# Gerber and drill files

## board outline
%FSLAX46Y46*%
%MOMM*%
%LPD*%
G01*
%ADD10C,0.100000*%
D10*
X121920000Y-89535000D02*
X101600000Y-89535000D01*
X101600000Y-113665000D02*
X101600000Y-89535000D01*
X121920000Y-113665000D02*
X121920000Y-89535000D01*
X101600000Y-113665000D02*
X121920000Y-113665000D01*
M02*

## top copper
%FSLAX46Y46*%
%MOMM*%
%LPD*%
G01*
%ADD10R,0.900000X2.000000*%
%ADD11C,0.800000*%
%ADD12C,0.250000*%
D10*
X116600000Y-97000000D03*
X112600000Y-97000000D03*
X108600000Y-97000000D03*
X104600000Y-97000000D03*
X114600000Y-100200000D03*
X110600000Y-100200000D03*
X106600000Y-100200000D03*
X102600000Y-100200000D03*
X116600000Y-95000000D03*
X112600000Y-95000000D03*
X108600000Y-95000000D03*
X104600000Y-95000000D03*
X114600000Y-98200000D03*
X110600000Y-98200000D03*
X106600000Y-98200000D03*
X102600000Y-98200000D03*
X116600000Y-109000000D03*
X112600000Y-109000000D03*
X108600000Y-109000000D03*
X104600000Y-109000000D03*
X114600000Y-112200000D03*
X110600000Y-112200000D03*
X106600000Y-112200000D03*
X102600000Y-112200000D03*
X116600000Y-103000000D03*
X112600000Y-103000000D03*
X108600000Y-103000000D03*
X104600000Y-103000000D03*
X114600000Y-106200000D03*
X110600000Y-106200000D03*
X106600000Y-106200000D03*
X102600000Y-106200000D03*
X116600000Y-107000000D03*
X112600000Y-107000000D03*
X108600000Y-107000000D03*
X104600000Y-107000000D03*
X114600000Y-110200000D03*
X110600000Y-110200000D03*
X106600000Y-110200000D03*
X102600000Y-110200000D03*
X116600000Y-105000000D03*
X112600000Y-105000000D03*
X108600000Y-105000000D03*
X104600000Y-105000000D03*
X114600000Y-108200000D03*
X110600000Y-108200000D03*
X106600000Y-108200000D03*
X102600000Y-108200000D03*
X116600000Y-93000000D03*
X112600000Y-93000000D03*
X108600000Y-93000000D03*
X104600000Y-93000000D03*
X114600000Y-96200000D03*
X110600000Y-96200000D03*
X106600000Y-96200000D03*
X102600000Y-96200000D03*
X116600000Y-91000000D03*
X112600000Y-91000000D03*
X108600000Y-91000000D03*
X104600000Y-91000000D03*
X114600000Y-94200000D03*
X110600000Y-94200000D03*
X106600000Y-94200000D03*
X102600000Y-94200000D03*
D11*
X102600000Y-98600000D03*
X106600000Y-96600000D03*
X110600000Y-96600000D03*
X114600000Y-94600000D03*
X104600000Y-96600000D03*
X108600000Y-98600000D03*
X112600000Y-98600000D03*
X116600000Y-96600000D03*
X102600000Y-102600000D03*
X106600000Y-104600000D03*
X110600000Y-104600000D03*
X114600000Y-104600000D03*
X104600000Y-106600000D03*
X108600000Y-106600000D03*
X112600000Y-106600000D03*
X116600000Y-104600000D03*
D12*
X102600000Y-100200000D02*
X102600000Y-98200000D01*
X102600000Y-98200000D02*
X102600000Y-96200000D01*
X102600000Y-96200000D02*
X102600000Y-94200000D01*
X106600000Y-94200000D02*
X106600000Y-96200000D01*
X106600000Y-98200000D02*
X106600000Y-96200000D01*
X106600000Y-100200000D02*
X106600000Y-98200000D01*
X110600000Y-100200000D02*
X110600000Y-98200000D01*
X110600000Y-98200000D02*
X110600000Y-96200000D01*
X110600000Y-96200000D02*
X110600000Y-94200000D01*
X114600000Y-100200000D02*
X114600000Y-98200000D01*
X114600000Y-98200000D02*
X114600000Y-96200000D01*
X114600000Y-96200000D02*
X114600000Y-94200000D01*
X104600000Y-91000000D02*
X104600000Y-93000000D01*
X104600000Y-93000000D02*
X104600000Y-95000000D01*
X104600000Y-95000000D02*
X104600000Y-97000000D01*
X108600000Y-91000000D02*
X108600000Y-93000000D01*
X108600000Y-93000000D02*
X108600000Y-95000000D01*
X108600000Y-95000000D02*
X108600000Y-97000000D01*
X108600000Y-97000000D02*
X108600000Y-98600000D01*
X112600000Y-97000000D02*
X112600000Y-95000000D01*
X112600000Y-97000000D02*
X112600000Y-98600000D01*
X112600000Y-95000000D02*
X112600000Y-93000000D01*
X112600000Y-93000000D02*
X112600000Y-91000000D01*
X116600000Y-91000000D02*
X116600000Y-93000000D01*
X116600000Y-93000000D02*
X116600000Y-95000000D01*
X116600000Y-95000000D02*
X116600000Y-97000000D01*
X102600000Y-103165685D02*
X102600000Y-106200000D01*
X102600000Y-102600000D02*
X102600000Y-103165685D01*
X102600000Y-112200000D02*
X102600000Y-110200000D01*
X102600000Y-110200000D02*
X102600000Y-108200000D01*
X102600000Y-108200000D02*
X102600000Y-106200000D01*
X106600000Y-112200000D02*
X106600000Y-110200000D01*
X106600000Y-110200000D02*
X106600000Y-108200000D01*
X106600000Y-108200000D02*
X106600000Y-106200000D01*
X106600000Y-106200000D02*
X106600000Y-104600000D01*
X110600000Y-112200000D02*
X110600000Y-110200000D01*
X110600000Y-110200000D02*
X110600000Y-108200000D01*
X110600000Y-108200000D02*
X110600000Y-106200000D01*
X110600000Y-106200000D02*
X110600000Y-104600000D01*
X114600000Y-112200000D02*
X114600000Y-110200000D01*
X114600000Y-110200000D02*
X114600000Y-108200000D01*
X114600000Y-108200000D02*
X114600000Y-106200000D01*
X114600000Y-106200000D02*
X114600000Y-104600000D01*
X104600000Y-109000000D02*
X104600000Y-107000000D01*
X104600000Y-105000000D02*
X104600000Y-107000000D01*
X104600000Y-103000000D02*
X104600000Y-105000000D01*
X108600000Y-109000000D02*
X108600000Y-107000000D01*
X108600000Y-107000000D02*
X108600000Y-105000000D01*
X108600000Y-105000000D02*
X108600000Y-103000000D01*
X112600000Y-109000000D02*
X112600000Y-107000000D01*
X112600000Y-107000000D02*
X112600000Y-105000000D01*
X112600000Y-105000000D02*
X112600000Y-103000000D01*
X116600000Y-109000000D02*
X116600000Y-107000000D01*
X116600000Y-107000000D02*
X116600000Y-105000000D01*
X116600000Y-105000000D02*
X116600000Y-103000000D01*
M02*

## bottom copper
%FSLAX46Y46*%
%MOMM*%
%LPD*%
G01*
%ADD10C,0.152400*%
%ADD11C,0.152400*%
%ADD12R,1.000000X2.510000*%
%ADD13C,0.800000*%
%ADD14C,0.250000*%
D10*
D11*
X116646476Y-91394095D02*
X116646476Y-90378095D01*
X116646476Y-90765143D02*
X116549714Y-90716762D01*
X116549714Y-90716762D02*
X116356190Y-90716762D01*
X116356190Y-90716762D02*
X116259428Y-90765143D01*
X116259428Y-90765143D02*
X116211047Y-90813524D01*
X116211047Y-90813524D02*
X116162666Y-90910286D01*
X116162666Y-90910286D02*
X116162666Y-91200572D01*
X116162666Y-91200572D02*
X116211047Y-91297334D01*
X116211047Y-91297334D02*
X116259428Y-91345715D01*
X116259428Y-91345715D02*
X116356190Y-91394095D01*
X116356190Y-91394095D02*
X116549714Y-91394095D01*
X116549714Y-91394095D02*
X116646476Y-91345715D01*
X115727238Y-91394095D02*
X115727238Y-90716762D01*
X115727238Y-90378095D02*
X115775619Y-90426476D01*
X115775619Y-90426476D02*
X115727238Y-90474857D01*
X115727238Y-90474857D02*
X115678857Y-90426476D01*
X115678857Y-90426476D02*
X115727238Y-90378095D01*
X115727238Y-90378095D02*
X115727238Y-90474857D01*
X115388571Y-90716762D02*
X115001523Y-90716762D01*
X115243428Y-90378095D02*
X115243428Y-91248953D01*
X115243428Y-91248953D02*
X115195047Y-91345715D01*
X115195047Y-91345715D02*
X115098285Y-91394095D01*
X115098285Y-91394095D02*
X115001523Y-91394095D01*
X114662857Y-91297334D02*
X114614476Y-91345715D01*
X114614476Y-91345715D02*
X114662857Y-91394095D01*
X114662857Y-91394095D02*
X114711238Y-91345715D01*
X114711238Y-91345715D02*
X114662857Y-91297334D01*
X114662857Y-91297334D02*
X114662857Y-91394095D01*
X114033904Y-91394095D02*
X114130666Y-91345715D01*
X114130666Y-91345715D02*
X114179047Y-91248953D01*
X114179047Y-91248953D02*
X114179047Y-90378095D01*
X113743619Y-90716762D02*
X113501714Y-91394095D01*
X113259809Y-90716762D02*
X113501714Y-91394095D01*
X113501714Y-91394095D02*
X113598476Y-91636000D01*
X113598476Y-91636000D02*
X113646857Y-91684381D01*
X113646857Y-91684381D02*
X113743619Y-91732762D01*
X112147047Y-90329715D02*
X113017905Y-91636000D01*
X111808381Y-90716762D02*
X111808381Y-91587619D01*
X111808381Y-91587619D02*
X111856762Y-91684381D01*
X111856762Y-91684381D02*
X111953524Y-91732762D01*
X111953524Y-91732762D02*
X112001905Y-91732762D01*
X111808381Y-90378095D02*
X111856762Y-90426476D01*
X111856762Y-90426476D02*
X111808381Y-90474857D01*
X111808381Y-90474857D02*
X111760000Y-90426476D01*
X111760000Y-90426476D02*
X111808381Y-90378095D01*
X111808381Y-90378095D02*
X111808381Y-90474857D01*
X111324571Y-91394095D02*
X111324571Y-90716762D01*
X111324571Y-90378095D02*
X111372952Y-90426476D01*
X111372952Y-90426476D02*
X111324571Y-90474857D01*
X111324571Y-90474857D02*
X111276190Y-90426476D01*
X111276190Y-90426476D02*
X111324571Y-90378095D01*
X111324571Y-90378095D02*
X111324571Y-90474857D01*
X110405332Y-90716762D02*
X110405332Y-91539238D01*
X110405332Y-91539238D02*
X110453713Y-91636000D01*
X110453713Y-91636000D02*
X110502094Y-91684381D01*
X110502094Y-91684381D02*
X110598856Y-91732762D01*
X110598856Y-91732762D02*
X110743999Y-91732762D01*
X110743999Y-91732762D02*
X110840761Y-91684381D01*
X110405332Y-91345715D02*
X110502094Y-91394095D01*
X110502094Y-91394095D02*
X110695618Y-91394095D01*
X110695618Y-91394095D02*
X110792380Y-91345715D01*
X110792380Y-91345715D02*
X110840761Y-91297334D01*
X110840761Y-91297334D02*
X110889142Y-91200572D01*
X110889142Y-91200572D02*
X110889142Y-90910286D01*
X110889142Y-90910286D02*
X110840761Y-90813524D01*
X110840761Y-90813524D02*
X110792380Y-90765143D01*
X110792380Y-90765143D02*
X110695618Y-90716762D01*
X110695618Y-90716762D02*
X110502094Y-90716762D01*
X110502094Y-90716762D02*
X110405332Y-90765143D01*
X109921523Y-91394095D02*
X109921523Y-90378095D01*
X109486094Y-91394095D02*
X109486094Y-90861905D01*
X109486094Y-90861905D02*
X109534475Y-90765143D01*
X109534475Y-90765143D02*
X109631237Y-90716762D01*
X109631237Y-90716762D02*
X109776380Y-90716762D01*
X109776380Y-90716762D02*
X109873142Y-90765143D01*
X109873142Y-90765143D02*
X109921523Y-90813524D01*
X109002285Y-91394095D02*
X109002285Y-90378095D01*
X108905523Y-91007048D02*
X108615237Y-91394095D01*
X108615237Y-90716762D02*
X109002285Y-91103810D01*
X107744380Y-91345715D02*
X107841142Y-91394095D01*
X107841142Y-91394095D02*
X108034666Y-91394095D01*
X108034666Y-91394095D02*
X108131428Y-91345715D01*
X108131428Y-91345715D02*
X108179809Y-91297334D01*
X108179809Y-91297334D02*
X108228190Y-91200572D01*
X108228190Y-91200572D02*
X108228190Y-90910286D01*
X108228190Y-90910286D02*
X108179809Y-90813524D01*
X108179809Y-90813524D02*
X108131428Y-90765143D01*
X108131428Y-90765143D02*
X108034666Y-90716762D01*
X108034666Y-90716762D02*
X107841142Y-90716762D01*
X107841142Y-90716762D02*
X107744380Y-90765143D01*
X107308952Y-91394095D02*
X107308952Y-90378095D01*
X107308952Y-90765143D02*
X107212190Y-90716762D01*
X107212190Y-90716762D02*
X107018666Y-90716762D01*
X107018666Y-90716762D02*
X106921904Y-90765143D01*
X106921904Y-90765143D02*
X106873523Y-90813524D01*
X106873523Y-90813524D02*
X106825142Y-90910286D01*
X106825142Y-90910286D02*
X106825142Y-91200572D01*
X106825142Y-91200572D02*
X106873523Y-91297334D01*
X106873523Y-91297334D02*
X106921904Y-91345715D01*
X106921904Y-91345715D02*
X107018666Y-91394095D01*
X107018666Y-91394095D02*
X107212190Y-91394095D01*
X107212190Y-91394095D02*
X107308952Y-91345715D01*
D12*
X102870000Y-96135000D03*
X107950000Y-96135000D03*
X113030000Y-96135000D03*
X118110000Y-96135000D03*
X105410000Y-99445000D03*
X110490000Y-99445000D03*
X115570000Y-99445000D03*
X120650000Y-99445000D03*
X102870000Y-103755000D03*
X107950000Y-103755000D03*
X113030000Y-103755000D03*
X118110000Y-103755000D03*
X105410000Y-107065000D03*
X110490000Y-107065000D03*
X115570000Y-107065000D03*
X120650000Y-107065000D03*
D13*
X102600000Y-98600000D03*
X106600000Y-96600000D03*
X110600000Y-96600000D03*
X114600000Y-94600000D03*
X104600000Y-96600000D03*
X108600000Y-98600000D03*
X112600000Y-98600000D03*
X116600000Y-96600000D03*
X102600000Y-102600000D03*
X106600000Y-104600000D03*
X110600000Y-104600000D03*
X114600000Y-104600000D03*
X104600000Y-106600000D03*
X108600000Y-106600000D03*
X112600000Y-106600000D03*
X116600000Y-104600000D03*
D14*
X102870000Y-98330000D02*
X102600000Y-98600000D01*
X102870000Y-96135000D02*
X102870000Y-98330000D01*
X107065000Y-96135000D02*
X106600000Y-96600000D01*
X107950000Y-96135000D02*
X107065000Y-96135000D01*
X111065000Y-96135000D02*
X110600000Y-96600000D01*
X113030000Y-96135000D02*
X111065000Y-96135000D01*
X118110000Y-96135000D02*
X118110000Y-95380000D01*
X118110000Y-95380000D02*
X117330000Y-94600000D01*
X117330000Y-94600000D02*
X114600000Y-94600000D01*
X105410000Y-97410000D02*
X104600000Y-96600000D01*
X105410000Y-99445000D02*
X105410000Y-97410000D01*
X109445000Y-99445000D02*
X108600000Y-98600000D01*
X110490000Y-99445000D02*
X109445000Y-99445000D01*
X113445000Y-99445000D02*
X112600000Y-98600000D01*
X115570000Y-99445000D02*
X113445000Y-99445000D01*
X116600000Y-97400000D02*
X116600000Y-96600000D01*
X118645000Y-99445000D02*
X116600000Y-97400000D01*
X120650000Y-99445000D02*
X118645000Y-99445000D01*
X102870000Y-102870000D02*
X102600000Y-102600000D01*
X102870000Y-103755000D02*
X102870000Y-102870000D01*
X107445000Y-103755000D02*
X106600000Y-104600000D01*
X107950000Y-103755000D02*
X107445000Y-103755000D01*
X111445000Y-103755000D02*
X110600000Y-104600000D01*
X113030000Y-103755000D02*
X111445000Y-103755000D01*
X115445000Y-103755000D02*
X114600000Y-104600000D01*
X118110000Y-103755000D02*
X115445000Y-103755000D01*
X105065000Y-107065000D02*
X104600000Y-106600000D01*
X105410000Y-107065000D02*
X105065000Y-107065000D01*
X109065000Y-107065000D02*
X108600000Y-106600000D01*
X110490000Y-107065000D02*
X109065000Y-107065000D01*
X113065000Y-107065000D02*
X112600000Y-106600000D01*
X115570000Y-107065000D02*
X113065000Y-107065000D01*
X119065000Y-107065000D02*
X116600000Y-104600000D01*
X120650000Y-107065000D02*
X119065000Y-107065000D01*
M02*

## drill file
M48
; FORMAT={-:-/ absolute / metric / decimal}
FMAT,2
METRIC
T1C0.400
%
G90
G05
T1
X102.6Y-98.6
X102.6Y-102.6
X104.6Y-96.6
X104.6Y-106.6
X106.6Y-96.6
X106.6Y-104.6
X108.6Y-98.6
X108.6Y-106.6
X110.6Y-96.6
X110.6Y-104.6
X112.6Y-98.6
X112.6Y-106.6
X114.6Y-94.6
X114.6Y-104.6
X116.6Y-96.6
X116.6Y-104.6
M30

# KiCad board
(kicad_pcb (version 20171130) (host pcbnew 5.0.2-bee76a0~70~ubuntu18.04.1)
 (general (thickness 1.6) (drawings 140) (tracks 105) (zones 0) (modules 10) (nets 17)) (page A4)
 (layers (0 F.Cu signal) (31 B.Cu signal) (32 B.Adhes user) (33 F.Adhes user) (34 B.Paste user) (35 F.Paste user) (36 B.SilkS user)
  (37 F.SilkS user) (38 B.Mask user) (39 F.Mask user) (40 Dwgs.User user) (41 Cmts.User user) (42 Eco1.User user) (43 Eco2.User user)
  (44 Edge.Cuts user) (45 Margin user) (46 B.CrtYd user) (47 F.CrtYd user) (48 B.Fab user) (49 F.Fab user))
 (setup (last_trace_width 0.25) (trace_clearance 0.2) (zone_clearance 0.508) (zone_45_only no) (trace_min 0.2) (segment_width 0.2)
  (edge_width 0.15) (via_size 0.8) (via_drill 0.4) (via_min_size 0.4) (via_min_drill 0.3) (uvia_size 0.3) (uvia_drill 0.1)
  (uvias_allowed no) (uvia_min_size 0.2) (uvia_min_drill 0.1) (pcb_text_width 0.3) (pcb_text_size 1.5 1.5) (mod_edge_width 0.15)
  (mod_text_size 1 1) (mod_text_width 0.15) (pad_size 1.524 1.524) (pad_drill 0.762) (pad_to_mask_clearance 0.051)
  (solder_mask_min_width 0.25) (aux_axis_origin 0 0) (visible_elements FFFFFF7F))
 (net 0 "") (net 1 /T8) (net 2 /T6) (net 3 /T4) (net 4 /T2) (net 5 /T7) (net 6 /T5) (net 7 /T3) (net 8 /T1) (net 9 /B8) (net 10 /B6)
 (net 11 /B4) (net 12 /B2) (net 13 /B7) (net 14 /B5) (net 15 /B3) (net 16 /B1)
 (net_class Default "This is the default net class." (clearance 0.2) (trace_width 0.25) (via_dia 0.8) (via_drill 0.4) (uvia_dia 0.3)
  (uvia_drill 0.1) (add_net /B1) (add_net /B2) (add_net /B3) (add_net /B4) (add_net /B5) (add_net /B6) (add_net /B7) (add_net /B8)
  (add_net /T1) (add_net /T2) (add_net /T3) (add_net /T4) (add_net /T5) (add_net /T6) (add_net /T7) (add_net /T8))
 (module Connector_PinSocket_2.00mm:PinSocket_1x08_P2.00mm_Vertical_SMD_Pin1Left (layer F.Cu) (at 109.6 98.6 90)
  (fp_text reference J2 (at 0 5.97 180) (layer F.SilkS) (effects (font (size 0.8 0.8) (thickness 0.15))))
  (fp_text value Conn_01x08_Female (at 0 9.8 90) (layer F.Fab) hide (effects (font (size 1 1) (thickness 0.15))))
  (pad 8 smd rect (at 1.6 7 90) (size 2 0.9) (layers F.Cu F.Paste F.Mask) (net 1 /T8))
  (pad 6 smd rect (at 1.6 3 90) (size 2 0.9) (layers F.Cu F.Paste F.Mask) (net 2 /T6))
  (pad 4 smd rect (at 1.6 -1 90) (size 2 0.9) (layers F.Cu F.Paste F.Mask) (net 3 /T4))
  (pad 2 smd rect (at 1.6 -5 90) (size 2 0.9) (layers F.Cu F.Paste F.Mask) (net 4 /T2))
  (pad 7 smd rect (at -1.6 5 90) (size 2 0.9) (layers F.Cu F.Paste F.Mask) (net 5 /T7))
  (pad 5 smd rect (at -1.6 1 90) (size 2 0.9) (layers F.Cu F.Paste F.Mask) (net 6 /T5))
  (pad 3 smd rect (at -1.6 -3 90) (size 2 0.9) (layers F.Cu F.Paste F.Mask) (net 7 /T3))
  (pad 1 smd rect (at -1.6 -7 90) (size 2 0.9) (layers F.Cu F.Paste F.Mask) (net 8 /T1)))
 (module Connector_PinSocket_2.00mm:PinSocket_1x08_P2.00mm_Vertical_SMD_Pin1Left (layer F.Cu) (at 109.6 96.6 90)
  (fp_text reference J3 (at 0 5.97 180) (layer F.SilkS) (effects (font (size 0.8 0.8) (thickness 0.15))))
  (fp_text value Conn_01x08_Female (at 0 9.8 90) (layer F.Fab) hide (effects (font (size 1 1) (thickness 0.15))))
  (pad 8 smd rect (at 1.6 7 90) (size 2 0.9) (layers F.Cu F.Paste F.Mask) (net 1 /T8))
  (pad 6 smd rect (at 1.6 3 90) (size 2 0.9) (layers F.Cu F.Paste F.Mask) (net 2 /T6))
  (pad 4 smd rect (at 1.6 -1 90) (size 2 0.9) (layers F.Cu F.Paste F.Mask) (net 3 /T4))
  (pad 2 smd rect (at 1.6 -5 90) (size 2 0.9) (layers F.Cu F.Paste F.Mask) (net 4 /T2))
  (pad 7 smd rect (at -1.6 5 90) (size 2 0.9) (layers F.Cu F.Paste F.Mask) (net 5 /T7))
  (pad 5 smd rect (at -1.6 1 90) (size 2 0.9) (layers F.Cu F.Paste F.Mask) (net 6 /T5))
  (pad 3 smd rect (at -1.6 -3 90) (size 2 0.9) (layers F.Cu F.Paste F.Mask) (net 7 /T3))
  (pad 1 smd rect (at -1.6 -7 90) (size 2 0.9) (layers F.Cu F.Paste F.Mask) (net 8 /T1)))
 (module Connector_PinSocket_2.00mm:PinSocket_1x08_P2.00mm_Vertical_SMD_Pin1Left (layer F.Cu) (at 109.6 110.6 90)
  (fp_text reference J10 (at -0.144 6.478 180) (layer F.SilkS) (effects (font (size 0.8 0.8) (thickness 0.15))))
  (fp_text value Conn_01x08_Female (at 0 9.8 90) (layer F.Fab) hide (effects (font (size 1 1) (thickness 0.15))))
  (pad 8 smd rect (at 1.6 7 90) (size 2 0.9) (layers F.Cu F.Paste F.Mask) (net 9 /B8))
  (pad 6 smd rect (at 1.6 3 90) (size 2 0.9) (layers F.Cu F.Paste F.Mask) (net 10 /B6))
  (pad 4 smd rect (at 1.6 -1 90) (size 2 0.9) (layers F.Cu F.Paste F.Mask) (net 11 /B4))
  (pad 2 smd rect (at 1.6 -5 90) (size 2 0.9) (layers F.Cu F.Paste F.Mask) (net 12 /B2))
  (pad 7 smd rect (at -1.6 5 90) (size 2 0.9) (layers F.Cu F.Paste F.Mask) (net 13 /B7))
  (pad 5 smd rect (at -1.6 1 90) (size 2 0.9) (layers F.Cu F.Paste F.Mask) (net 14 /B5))
  (pad 3 smd rect (at -1.6 -3 90) (size 2 0.9) (layers F.Cu F.Paste F.Mask) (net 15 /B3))
  (pad 1 smd rect (at -1.6 -7 90) (size 2 0.9) (layers F.Cu F.Paste F.Mask) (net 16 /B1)))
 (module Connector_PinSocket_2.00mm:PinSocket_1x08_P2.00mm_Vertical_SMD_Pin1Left (layer F.Cu) (at 109.6 104.6 90)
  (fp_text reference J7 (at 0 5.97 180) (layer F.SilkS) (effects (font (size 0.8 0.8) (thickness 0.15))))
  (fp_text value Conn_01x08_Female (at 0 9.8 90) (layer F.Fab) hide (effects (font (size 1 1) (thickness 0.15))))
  (pad 8 smd rect (at 1.6 7 90) (size 2 0.9) (layers F.Cu F.Paste F.Mask) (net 9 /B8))
  (pad 6 smd rect (at 1.6 3 90) (size 2 0.9) (layers F.Cu F.Paste F.Mask) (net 10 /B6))
  (pad 4 smd rect (at 1.6 -1 90) (size 2 0.9) (layers F.Cu F.Paste F.Mask) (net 11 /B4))
  (pad 2 smd rect (at 1.6 -5 90) (size 2 0.9) (layers F.Cu F.Paste F.Mask) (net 12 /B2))
  (pad 7 smd rect (at -1.6 5 90) (size 2 0.9) (layers F.Cu F.Paste F.Mask) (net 13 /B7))
  (pad 5 smd rect (at -1.6 1 90) (size 2 0.9) (layers F.Cu F.Paste F.Mask) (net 14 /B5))
  (pad 3 smd rect (at -1.6 -3 90) (size 2 0.9) (layers F.Cu F.Paste F.Mask) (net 15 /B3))
  (pad 1 smd rect (at -1.6 -7 90) (size 2 0.9) (layers F.Cu F.Paste F.Mask) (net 16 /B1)))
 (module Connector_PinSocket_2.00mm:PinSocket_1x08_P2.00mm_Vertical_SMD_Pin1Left (layer F.Cu) (at 109.6 108.6 90)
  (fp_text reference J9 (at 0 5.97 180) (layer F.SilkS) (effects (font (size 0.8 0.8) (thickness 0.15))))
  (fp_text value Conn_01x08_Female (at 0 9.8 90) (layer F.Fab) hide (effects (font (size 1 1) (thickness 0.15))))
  (pad 8 smd rect (at 1.6 7 90) (size 2 0.9) (layers F.Cu F.Paste F.Mask) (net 9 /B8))
  (pad 6 smd rect (at 1.6 3 90) (size 2 0.9) (layers F.Cu F.Paste F.Mask) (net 10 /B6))
  (pad 4 smd rect (at 1.6 -1 90) (size 2 0.9) (layers F.Cu F.Paste F.Mask) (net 11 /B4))
  (pad 2 smd rect (at 1.6 -5 90) (size 2 0.9) (layers F.Cu F.Paste F.Mask) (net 12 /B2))
  (pad 7 smd rect (at -1.6 5 90) (size 2 0.9) (layers F.Cu F.Paste F.Mask) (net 13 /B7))
  (pad 5 smd rect (at -1.6 1 90) (size 2 0.9) (layers F.Cu F.Paste F.Mask) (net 14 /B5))
  (pad 3 smd rect (at -1.6 -3 90) (size 2 0.9) (layers F.Cu F.Paste F.Mask) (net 15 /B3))
  (pad 1 smd rect (at -1.6 -7 90) (size 2 0.9) (layers F.Cu F.Paste F.Mask) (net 16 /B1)))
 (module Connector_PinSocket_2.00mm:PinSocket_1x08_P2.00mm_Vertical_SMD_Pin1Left (layer F.Cu) (at 109.6 106.6 90)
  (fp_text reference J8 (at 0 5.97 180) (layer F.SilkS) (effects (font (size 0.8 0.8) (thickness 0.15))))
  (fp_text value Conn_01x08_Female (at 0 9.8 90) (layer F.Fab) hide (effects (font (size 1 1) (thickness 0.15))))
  (pad 8 smd rect (at 1.6 7 90) (size 2 0.9) (layers F.Cu F.Paste F.Mask) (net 9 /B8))
  (pad 6 smd rect (at 1.6 3 90) (size 2 0.9) (layers F.Cu F.Paste F.Mask) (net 10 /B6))
  (pad 4 smd rect (at 1.6 -1 90) (size 2 0.9) (layers F.Cu F.Paste F.Mask) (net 11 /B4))
  (pad 2 smd rect (at 1.6 -5 90) (size 2 0.9) (layers F.Cu F.Paste F.Mask) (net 12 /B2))
  (pad 7 smd rect (at -1.6 5 90) (size 2 0.9) (layers F.Cu F.Paste F.Mask) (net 13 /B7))
  (pad 5 smd rect (at -1.6 1 90) (size 2 0.9) (layers F.Cu F.Paste F.Mask) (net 14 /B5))
  (pad 3 smd rect (at -1.6 -3 90) (size 2 0.9) (layers F.Cu F.Paste F.Mask) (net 15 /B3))
  (pad 1 smd rect (at -1.6 -7 90) (size 2 0.9) (layers F.Cu F.Paste F.Mask) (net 16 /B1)))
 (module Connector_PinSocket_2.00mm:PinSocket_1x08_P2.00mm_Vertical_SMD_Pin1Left (layer F.Cu) (at 109.6 94.6 90)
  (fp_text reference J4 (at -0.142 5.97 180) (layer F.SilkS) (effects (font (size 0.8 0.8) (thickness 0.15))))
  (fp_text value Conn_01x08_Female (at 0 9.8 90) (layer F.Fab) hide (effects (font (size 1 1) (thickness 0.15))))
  (pad 8 smd rect (at 1.6 7 90) (size 2 0.9) (layers F.Cu F.Paste F.Mask) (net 1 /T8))
  (pad 6 smd rect (at 1.6 3 90) (size 2 0.9) (layers F.Cu F.Paste F.Mask) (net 2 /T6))
  (pad 4 smd rect (at 1.6 -1 90) (size 2 0.9) (layers F.Cu F.Paste F.Mask) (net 3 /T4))
  (pad 2 smd rect (at 1.6 -5 90) (size 2 0.9) (layers F.Cu F.Paste F.Mask) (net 4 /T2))
  (pad 7 smd rect (at -1.6 5 90) (size 2 0.9) (layers F.Cu F.Paste F.Mask) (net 5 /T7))
  (pad 5 smd rect (at -1.6 1 90) (size 2 0.9) (layers F.Cu F.Paste F.Mask) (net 6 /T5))
  (pad 3 smd rect (at -1.6 -3 90) (size 2 0.9) (layers F.Cu F.Paste F.Mask) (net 7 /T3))
  (pad 1 smd rect (at -1.6 -7 90) (size 2 0.9) (layers F.Cu F.Paste F.Mask) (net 8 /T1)))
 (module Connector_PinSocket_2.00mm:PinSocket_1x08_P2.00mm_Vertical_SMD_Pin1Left (layer F.Cu) (at 109.6 92.6 90)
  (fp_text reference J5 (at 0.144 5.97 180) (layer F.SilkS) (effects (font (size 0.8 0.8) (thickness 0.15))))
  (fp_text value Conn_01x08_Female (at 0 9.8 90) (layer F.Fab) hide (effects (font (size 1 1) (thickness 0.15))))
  (pad 8 smd rect (at 1.6 7 90) (size 2 0.9) (layers F.Cu F.Paste F.Mask) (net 1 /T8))
  (pad 6 smd rect (at 1.6 3 90) (size 2 0.9) (layers F.Cu F.Paste F.Mask) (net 2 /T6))
  (pad 4 smd rect (at 1.6 -1 90) (size 2 0.9) (layers F.Cu F.Paste F.Mask) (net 3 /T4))
  (pad 2 smd rect (at 1.6 -5 90) (size 2 0.9) (layers F.Cu F.Paste F.Mask) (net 4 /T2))
  (pad 7 smd rect (at -1.6 5 90) (size 2 0.9) (layers F.Cu F.Paste F.Mask) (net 5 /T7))
  (pad 5 smd rect (at -1.6 1 90) (size 2 0.9) (layers F.Cu F.Paste F.Mask) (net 6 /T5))
  (pad 3 smd rect (at -1.6 -3 90) (size 2 0.9) (layers F.Cu F.Paste F.Mask) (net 7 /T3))
  (pad 1 smd rect (at -1.6 -7 90) (size 2 0.9) (layers F.Cu F.Paste F.Mask) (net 8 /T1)))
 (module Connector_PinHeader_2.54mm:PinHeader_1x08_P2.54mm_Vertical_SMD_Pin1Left (layer B.Cu) (at 111.76 97.79 270)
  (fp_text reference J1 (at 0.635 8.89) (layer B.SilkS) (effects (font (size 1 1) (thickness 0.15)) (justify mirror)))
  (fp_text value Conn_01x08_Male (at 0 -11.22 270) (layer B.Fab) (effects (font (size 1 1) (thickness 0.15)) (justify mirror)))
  (pad 1 smd rect (at -1.655 8.89 270) (size 2.51 1) (layers B.Cu B.Paste B.Mask) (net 8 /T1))
  (pad 3 smd rect (at -1.655 3.81 270) (size 2.51 1) (layers B.Cu B.Paste B.Mask) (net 7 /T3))
  (pad 5 smd rect (at -1.655 -1.27 270) (size 2.51 1) (layers B.Cu B.Paste B.Mask) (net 6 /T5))
  (pad 7 smd rect (at -1.655 -6.35 270) (size 2.51 1) (layers B.Cu B.Paste B.Mask) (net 5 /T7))
  (pad 2 smd rect (at 1.655 6.35 270) (size 2.51 1) (layers B.Cu B.Paste B.Mask) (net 4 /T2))
  (pad 4 smd rect (at 1.655 1.27 270) (size 2.51 1) (layers B.Cu B.Paste B.Mask) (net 3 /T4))
  (pad 6 smd rect (at 1.655 -3.81 270) (size 2.51 1) (layers B.Cu B.Paste B.Mask) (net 2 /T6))
  (pad 8 smd rect (at 1.655 -8.89 270) (size 2.51 1) (layers B.Cu B.Paste B.Mask) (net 1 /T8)))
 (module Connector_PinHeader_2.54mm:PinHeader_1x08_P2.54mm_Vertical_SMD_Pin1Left (layer B.Cu) (at 111.76 105.41 270)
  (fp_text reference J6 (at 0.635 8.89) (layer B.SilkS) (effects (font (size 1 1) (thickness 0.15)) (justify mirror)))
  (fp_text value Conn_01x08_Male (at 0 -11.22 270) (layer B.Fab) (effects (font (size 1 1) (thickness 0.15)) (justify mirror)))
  (pad 1 smd rect (at -1.655 8.89 270) (size 2.51 1) (layers B.Cu B.Paste B.Mask) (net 16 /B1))
  (pad 3 smd rect (at -1.655 3.81 270) (size 2.51 1) (layers B.Cu B.Paste B.Mask) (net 15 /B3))
  (pad 5 smd rect (at -1.655 -1.27 270) (size 2.51 1) (layers B.Cu B.Paste B.Mask) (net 14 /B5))
  (pad 7 smd rect (at -1.655 -6.35 270) (size 2.51 1) (layers B.Cu B.Paste B.Mask) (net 13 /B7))
  (pad 2 smd rect (at 1.655 6.35 270) (size 2.51 1) (layers B.Cu B.Paste B.Mask) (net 12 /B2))
  (pad 4 smd rect (at 1.655 1.27 270) (size 2.51 1) (layers B.Cu B.Paste B.Mask) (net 11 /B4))
  (pad 6 smd rect (at 1.655 -3.81 270) (size 2.51 1) (layers B.Cu B.Paste B.Mask) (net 10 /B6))
  (pad 8 smd rect (at 1.655 -8.89 270) (size 2.51 1) (layers B.Cu B.Paste B.Mask) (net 9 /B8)))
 (gr_line (start 121.92 89.535) (end 101.6 89.535) (layer Edge.Cuts) (width 0.1))
 (gr_line (start 101.6 113.665) (end 101.6 89.535) (layer Edge.Cuts) (width 0.1))
 (gr_line (start 121.92 113.665) (end 121.92 89.535) (layer Edge.Cuts) (width 0.1))
 (gr_line (start 101.6 113.665) (end 121.92 113.665) (layer Edge.Cuts) (width 0.1))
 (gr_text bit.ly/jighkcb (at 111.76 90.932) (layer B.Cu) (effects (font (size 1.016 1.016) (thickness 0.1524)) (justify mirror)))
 (via (at 102.6 98.6) (size 0.8) (drill 0.4) (layers F.Cu B.Cu) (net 8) (status 30))
 (segment (start 102.87 98.33) (end 102.6 98.6) (width 0.25) (layer B.Cu) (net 8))
 (segment (start 102.87 96.135) (end 102.87 98.33) (width 0.25) (layer B.Cu) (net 8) (status 10))
 (segment (start 102.6 100.2) (end 102.6 98.2) (width 0.25) (layer F.Cu) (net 8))
 (segment (start 102.6 98.2) (end 102.6 96.2) (width 0.25) (layer F.Cu) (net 8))
 (segment (start 102.6 96.2) (end 102.6 94.2) (width 0.25) (layer F.Cu) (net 8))
 (via (at 106.6 96.6) (size 0.8) (drill 0.4) (layers F.Cu B.Cu) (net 7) (status 30))
 (segment (start 107.065 96.135) (end 106.6 96.6) (width 0.25) (layer B.Cu) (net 7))
 (segment (start 107.95 96.135) (end 107.065 96.135) (width 0.25) (layer B.Cu) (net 7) (status 10))
 (segment (start 106.6 94.2) (end 106.6 96.2) (width 0.25) (layer F.Cu) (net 7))
 (segment (start 106.6 98.2) (end 106.6 96.2) (width 0.25) (layer F.Cu) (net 7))
 (segment (start 106.6 100.2) (end 106.6 98.2) (width 0.25) (layer F.Cu) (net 7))
 (via (at 110.6 96.6) (size 0.8) (drill 0.4) (layers F.Cu B.Cu) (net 6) (status 30))
 (segment (start 111.065 96.135) (end 110.6 96.6) (width 0.25) (layer B.Cu) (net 6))
 (segment (start 113.03 96.135) (end 111.065 96.135) (width 0.25) (layer B.Cu) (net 6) (status 10))
 (segment (start 110.6 100.2) (end 110.6 98.2) (width 0.25) (layer F.Cu) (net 6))
 (segment (start 110.6 98.2) (end 110.6 96.2) (width 0.25) (layer F.Cu) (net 6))
 (segment (start 110.6 96.2) (end 110.6 94.2) (width 0.25) (layer F.Cu) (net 6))
 (segment (start 118.11 96.135) (end 118.11 95.38) (width 0.25) (layer B.Cu) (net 5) (status 30))
 (segment (start 118.11 95.38) (end 117.33 94.6) (width 0.25) (layer B.Cu) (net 5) (status 10))
 (via (at 114.6 94.6) (size 0.8) (drill 0.4) (layers F.Cu B.Cu) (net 5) (status 30))
 (segment (start 117.33 94.6) (end 114.6 94.6) (width 0.25) (layer B.Cu) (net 5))
 (segment (start 114.6 100.2) (end 114.6 98.2) (width 0.25) (layer F.Cu) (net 5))
 (segment (start 114.6 98.2) (end 114.6 96.2) (width 0.25) (layer F.Cu) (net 5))
 (segment (start 114.6 96.2) (end 114.6 94.2) (width 0.25) (layer F.Cu) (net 5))
 (via (at 104.6 96.6) (size 0.8) (drill 0.4) (layers F.Cu B.Cu) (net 4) (status 30))
 (segment (start 105.41 97.41) (end 104.6 96.6) (width 0.25) (layer B.Cu) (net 4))
 (segment (start 105.41 99.445) (end 105.41 97.41) (width 0.25) (layer B.Cu) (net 4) (status 10))
 (segment (start 104.6 91) (end 104.6 93) (width 0.25) (layer F.Cu) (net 4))
 (segment (start 104.6 93) (end 104.6 95) (width 0.25) (layer F.Cu) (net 4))
 (segment (start 104.6 95) (end 104.6 97) (width 0.25) (layer F.Cu) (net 4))
 (via (at 108.6 98.6) (size 0.8) (drill 0.4) (layers F.Cu B.Cu) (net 3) (status 30))
 (segment (start 109.445 99.445) (end 108.6 98.6) (width 0.25) (layer B.Cu) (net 3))
 (segment (start 110.49 99.445) (end 109.445 99.445) (width 0.25) (layer B.Cu) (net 3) (status 10))
 (segment (start 108.6 91) (end 108.6 93) (width 0.25) (layer F.Cu) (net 3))
 (segment (start 108.6 93) (end 108.6 95) (width 0.25) (layer F.Cu) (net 3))
 (segment (start 108.6 95) (end 108.6 97) (width 0.25) (layer F.Cu) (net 3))
 (segment (start 108.6 97) (end 108.6 98.6) (width 0.25) (layer F.Cu) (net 3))
 (via (at 112.6 98.6) (size 0.8) (drill 0.4) (layers F.Cu B.Cu) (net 2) (status 30))
 (segment (start 113.445 99.445) (end 112.6 98.6) (width 0.25) (layer B.Cu) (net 2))
 (segment (start 115.57 99.445) (end 113.445 99.445) (width 0.25) (layer B.Cu) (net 2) (status 10))
 (segment (start 112.6 97) (end 112.6 95) (width 0.25) (layer F.Cu) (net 2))
 (segment (start 112.6 97) (end 112.6 98.6) (width 0.25) (layer F.Cu) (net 2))
 (segment (start 112.6 95) (end 112.6 93) (width 0.25) (layer F.Cu) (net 2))
 (segment (start 112.6 93) (end 112.6 91) (width 0.25) (layer F.Cu) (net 2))
 (via (at 116.6 96.6) (size 0.8) (drill 0.4) (layers F.Cu B.Cu) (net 1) (status 30))
 (segment (start 116.6 97.4) (end 116.6 96.6) (width 0.25) (layer B.Cu) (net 1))
 (segment (start 118.645 99.445) (end 116.6 97.4) (width 0.25) (layer B.Cu) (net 1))
 (segment (start 120.65 99.445) (end 118.645 99.445) (width 0.25) (layer B.Cu) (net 1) (status 10))
 (segment (start 116.6 91) (end 116.6 93) (width 0.25) (layer F.Cu) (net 1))
 (segment (start 116.6 93) (end 116.6 95) (width 0.25) (layer F.Cu) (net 1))
 (segment (start 116.6 95) (end 116.6 97) (width 0.25) (layer F.Cu) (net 1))
 (via (at 102.6 102.6) (size 0.8) (drill 0.4) (layers F.Cu B.Cu) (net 16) (status 30))
 (segment (start 102.87 102.87) (end 102.6 102.6) (width 0.25) (layer B.Cu) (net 16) (status 30))
 (segment (start 102.87 103.755) (end 102.87 102.87) (width 0.25) (layer B.Cu) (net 16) (status 30))
 (segment (start 102.6 103.165685) (end 102.6 106.2) (width 0.25) (layer F.Cu) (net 16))
 (segment (start 102.6 102.6) (end 102.6 103.165685) (width 0.25) (layer F.Cu) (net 16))
 (segment (start 102.6 112.2) (end 102.6 110.2) (width 0.25) (layer F.Cu) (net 16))
 (segment (start 102.6 110.2) (end 102.6 108.2) (width 0.25) (layer F.Cu) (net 16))
 (segment (start 102.6 108.2) (end 102.6 106.2) (width 0.25) (layer F.Cu) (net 16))
 (via (at 106.6 104.6) (size 0.8) (drill 0.4) (layers F.Cu B.Cu) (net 15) (status 30))
 (segment (start 107.445 103.755) (end 106.6 104.6) (width 0.25) (layer B.Cu) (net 15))
 (segment (start 107.95 103.755) (end 107.445 103.755) (width 0.25) (layer B.Cu) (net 15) (status 10))
 (segment (start 106.6 112.2) (end 106.6 110.2) (width 0.25) (layer F.Cu) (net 15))
 (segment (start 106.6 110.2) (end 106.6 108.2) (width 0.25) (layer F.Cu) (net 15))
 (segment (start 106.6 108.2) (end 106.6 106.2) (width 0.25) (layer F.Cu) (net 15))
 (segment (start 106.6 106.2) (end 106.6 104.6) (width 0.25) (layer F.Cu) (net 15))
 (via (at 110.6 104.6) (size 0.8) (drill 0.4) (layers F.Cu B.Cu) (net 14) (status 30))
 (segment (start 111.445 103.755) (end 110.6 104.6) (width 0.25) (layer B.Cu) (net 14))
 (segment (start 113.03 103.755) (end 111.445 103.755) (width 0.25) (layer B.Cu) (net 14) (status 10))
 (segment (start 110.6 112.2) (end 110.6 110.2) (width 0.25) (layer F.Cu) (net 14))
 (segment (start 110.6 110.2) (end 110.6 108.2) (width 0.25) (layer F.Cu) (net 14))
 (segment (start 110.6 108.2) (end 110.6 106.2) (width 0.25) (layer F.Cu) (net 14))
 (segment (start 110.6 106.2) (end 110.6 104.6) (width 0.25) (layer F.Cu) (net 14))
 (via (at 114.6 104.6) (size 0.8) (drill 0.4) (layers F.Cu B.Cu) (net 13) (status 30))
 (segment (start 115.445 103.755) (end 114.6 104.6) (width 0.25) (layer B.Cu) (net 13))
 (segment (start 118.11 103.755) (end 115.445 103.755) (width 0.25) (layer B.Cu) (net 13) (status 10))
 (segment (start 114.6 112.2) (end 114.6 110.2) (width 0.25) (layer F.Cu) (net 13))
 (segment (start 114.6 110.2) (end 114.6 108.2) (width 0.25) (layer F.Cu) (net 13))
 (segment (start 114.6 108.2) (end 114.6 106.2) (width 0.25) (layer F.Cu) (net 13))
 (segment (start 114.6 106.2) (end 114.6 104.6) (width 0.25) (layer F.Cu) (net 13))
 (via (at 104.6 106.6) (size 0.8) (drill 0.4) (layers F.Cu B.Cu) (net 12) (status 30))
 (segment (start 105.065 107.065) (end 104.6 106.6) (width 0.25) (layer B.Cu) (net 12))
 (segment (start 105.41 107.065) (end 105.065 107.065) (width 0.25) (layer B.Cu) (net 12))
 (segment (start 104.6 109) (end 104.6 107) (width 0.25) (layer F.Cu) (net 12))
 (segment (start 104.6 105) (end 104.6 107) (width 0.25) (layer F.Cu) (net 12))
 (segment (start 104.6 103) (end 104.6 105) (width 0.25) (layer F.Cu) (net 12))
 (via (at 108.6 106.6) (size 0.8) (drill 0.4) (layers F.Cu B.Cu) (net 11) (status 30))
 (segment (start 109.065 107.065) (end 108.6 106.6) (width 0.25) (layer B.Cu) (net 11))
 (segment (start 110.49 107.065) (end 109.065 107.065) (width 0.25) (layer B.Cu) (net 11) (status 10))
 (segment (start 108.6 109) (end 108.6 107) (width 0.25) (layer F.Cu) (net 11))
 (segment (start 108.6 107) (end 108.6 105) (width 0.25) (layer F.Cu) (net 11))
 (segment (start 108.6 105) (end 108.6 103) (width 0.25) (layer F.Cu) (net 11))
 (via (at 112.6 106.6) (size 0.8) (drill 0.4) (layers F.Cu B.Cu) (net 10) (status 30))
 (segment (start 113.065 107.065) (end 112.6 106.6) (width 0.25) (layer B.Cu) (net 10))
 (segment (start 115.57 107.065) (end 113.065 107.065) (width 0.25) (layer B.Cu) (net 10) (status 10))
 (segment (start 112.6 109) (end 112.6 107) (width 0.25) (layer F.Cu) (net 10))
 (segment (start 112.6 107) (end 112.6 105) (width 0.25) (layer F.Cu) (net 10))
 (segment (start 112.6 105) (end 112.6 103) (width 0.25) (layer F.Cu) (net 10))
 (via (at 116.6 104.6) (size 0.8) (drill 0.4) (layers F.Cu B.Cu) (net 9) (status 30))
 (segment (start 119.065 107.065) (end 116.6 104.6) (width 0.25) (layer B.Cu) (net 9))
 (segment (start 120.65 107.065) (end 119.065 107.065) (width 0.25) (layer B.Cu) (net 9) (status 10))
 (segment (start 116.6 109) (end 116.6 107) (width 0.25) (layer F.Cu) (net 9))
 (segment (start 116.6 107) (end 116.6 105) (width 0.25) (layer F.Cu) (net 9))
 (segment (start 116.6 105) (end 116.6 103) (width 0.25) (layer F.Cu) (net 9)))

